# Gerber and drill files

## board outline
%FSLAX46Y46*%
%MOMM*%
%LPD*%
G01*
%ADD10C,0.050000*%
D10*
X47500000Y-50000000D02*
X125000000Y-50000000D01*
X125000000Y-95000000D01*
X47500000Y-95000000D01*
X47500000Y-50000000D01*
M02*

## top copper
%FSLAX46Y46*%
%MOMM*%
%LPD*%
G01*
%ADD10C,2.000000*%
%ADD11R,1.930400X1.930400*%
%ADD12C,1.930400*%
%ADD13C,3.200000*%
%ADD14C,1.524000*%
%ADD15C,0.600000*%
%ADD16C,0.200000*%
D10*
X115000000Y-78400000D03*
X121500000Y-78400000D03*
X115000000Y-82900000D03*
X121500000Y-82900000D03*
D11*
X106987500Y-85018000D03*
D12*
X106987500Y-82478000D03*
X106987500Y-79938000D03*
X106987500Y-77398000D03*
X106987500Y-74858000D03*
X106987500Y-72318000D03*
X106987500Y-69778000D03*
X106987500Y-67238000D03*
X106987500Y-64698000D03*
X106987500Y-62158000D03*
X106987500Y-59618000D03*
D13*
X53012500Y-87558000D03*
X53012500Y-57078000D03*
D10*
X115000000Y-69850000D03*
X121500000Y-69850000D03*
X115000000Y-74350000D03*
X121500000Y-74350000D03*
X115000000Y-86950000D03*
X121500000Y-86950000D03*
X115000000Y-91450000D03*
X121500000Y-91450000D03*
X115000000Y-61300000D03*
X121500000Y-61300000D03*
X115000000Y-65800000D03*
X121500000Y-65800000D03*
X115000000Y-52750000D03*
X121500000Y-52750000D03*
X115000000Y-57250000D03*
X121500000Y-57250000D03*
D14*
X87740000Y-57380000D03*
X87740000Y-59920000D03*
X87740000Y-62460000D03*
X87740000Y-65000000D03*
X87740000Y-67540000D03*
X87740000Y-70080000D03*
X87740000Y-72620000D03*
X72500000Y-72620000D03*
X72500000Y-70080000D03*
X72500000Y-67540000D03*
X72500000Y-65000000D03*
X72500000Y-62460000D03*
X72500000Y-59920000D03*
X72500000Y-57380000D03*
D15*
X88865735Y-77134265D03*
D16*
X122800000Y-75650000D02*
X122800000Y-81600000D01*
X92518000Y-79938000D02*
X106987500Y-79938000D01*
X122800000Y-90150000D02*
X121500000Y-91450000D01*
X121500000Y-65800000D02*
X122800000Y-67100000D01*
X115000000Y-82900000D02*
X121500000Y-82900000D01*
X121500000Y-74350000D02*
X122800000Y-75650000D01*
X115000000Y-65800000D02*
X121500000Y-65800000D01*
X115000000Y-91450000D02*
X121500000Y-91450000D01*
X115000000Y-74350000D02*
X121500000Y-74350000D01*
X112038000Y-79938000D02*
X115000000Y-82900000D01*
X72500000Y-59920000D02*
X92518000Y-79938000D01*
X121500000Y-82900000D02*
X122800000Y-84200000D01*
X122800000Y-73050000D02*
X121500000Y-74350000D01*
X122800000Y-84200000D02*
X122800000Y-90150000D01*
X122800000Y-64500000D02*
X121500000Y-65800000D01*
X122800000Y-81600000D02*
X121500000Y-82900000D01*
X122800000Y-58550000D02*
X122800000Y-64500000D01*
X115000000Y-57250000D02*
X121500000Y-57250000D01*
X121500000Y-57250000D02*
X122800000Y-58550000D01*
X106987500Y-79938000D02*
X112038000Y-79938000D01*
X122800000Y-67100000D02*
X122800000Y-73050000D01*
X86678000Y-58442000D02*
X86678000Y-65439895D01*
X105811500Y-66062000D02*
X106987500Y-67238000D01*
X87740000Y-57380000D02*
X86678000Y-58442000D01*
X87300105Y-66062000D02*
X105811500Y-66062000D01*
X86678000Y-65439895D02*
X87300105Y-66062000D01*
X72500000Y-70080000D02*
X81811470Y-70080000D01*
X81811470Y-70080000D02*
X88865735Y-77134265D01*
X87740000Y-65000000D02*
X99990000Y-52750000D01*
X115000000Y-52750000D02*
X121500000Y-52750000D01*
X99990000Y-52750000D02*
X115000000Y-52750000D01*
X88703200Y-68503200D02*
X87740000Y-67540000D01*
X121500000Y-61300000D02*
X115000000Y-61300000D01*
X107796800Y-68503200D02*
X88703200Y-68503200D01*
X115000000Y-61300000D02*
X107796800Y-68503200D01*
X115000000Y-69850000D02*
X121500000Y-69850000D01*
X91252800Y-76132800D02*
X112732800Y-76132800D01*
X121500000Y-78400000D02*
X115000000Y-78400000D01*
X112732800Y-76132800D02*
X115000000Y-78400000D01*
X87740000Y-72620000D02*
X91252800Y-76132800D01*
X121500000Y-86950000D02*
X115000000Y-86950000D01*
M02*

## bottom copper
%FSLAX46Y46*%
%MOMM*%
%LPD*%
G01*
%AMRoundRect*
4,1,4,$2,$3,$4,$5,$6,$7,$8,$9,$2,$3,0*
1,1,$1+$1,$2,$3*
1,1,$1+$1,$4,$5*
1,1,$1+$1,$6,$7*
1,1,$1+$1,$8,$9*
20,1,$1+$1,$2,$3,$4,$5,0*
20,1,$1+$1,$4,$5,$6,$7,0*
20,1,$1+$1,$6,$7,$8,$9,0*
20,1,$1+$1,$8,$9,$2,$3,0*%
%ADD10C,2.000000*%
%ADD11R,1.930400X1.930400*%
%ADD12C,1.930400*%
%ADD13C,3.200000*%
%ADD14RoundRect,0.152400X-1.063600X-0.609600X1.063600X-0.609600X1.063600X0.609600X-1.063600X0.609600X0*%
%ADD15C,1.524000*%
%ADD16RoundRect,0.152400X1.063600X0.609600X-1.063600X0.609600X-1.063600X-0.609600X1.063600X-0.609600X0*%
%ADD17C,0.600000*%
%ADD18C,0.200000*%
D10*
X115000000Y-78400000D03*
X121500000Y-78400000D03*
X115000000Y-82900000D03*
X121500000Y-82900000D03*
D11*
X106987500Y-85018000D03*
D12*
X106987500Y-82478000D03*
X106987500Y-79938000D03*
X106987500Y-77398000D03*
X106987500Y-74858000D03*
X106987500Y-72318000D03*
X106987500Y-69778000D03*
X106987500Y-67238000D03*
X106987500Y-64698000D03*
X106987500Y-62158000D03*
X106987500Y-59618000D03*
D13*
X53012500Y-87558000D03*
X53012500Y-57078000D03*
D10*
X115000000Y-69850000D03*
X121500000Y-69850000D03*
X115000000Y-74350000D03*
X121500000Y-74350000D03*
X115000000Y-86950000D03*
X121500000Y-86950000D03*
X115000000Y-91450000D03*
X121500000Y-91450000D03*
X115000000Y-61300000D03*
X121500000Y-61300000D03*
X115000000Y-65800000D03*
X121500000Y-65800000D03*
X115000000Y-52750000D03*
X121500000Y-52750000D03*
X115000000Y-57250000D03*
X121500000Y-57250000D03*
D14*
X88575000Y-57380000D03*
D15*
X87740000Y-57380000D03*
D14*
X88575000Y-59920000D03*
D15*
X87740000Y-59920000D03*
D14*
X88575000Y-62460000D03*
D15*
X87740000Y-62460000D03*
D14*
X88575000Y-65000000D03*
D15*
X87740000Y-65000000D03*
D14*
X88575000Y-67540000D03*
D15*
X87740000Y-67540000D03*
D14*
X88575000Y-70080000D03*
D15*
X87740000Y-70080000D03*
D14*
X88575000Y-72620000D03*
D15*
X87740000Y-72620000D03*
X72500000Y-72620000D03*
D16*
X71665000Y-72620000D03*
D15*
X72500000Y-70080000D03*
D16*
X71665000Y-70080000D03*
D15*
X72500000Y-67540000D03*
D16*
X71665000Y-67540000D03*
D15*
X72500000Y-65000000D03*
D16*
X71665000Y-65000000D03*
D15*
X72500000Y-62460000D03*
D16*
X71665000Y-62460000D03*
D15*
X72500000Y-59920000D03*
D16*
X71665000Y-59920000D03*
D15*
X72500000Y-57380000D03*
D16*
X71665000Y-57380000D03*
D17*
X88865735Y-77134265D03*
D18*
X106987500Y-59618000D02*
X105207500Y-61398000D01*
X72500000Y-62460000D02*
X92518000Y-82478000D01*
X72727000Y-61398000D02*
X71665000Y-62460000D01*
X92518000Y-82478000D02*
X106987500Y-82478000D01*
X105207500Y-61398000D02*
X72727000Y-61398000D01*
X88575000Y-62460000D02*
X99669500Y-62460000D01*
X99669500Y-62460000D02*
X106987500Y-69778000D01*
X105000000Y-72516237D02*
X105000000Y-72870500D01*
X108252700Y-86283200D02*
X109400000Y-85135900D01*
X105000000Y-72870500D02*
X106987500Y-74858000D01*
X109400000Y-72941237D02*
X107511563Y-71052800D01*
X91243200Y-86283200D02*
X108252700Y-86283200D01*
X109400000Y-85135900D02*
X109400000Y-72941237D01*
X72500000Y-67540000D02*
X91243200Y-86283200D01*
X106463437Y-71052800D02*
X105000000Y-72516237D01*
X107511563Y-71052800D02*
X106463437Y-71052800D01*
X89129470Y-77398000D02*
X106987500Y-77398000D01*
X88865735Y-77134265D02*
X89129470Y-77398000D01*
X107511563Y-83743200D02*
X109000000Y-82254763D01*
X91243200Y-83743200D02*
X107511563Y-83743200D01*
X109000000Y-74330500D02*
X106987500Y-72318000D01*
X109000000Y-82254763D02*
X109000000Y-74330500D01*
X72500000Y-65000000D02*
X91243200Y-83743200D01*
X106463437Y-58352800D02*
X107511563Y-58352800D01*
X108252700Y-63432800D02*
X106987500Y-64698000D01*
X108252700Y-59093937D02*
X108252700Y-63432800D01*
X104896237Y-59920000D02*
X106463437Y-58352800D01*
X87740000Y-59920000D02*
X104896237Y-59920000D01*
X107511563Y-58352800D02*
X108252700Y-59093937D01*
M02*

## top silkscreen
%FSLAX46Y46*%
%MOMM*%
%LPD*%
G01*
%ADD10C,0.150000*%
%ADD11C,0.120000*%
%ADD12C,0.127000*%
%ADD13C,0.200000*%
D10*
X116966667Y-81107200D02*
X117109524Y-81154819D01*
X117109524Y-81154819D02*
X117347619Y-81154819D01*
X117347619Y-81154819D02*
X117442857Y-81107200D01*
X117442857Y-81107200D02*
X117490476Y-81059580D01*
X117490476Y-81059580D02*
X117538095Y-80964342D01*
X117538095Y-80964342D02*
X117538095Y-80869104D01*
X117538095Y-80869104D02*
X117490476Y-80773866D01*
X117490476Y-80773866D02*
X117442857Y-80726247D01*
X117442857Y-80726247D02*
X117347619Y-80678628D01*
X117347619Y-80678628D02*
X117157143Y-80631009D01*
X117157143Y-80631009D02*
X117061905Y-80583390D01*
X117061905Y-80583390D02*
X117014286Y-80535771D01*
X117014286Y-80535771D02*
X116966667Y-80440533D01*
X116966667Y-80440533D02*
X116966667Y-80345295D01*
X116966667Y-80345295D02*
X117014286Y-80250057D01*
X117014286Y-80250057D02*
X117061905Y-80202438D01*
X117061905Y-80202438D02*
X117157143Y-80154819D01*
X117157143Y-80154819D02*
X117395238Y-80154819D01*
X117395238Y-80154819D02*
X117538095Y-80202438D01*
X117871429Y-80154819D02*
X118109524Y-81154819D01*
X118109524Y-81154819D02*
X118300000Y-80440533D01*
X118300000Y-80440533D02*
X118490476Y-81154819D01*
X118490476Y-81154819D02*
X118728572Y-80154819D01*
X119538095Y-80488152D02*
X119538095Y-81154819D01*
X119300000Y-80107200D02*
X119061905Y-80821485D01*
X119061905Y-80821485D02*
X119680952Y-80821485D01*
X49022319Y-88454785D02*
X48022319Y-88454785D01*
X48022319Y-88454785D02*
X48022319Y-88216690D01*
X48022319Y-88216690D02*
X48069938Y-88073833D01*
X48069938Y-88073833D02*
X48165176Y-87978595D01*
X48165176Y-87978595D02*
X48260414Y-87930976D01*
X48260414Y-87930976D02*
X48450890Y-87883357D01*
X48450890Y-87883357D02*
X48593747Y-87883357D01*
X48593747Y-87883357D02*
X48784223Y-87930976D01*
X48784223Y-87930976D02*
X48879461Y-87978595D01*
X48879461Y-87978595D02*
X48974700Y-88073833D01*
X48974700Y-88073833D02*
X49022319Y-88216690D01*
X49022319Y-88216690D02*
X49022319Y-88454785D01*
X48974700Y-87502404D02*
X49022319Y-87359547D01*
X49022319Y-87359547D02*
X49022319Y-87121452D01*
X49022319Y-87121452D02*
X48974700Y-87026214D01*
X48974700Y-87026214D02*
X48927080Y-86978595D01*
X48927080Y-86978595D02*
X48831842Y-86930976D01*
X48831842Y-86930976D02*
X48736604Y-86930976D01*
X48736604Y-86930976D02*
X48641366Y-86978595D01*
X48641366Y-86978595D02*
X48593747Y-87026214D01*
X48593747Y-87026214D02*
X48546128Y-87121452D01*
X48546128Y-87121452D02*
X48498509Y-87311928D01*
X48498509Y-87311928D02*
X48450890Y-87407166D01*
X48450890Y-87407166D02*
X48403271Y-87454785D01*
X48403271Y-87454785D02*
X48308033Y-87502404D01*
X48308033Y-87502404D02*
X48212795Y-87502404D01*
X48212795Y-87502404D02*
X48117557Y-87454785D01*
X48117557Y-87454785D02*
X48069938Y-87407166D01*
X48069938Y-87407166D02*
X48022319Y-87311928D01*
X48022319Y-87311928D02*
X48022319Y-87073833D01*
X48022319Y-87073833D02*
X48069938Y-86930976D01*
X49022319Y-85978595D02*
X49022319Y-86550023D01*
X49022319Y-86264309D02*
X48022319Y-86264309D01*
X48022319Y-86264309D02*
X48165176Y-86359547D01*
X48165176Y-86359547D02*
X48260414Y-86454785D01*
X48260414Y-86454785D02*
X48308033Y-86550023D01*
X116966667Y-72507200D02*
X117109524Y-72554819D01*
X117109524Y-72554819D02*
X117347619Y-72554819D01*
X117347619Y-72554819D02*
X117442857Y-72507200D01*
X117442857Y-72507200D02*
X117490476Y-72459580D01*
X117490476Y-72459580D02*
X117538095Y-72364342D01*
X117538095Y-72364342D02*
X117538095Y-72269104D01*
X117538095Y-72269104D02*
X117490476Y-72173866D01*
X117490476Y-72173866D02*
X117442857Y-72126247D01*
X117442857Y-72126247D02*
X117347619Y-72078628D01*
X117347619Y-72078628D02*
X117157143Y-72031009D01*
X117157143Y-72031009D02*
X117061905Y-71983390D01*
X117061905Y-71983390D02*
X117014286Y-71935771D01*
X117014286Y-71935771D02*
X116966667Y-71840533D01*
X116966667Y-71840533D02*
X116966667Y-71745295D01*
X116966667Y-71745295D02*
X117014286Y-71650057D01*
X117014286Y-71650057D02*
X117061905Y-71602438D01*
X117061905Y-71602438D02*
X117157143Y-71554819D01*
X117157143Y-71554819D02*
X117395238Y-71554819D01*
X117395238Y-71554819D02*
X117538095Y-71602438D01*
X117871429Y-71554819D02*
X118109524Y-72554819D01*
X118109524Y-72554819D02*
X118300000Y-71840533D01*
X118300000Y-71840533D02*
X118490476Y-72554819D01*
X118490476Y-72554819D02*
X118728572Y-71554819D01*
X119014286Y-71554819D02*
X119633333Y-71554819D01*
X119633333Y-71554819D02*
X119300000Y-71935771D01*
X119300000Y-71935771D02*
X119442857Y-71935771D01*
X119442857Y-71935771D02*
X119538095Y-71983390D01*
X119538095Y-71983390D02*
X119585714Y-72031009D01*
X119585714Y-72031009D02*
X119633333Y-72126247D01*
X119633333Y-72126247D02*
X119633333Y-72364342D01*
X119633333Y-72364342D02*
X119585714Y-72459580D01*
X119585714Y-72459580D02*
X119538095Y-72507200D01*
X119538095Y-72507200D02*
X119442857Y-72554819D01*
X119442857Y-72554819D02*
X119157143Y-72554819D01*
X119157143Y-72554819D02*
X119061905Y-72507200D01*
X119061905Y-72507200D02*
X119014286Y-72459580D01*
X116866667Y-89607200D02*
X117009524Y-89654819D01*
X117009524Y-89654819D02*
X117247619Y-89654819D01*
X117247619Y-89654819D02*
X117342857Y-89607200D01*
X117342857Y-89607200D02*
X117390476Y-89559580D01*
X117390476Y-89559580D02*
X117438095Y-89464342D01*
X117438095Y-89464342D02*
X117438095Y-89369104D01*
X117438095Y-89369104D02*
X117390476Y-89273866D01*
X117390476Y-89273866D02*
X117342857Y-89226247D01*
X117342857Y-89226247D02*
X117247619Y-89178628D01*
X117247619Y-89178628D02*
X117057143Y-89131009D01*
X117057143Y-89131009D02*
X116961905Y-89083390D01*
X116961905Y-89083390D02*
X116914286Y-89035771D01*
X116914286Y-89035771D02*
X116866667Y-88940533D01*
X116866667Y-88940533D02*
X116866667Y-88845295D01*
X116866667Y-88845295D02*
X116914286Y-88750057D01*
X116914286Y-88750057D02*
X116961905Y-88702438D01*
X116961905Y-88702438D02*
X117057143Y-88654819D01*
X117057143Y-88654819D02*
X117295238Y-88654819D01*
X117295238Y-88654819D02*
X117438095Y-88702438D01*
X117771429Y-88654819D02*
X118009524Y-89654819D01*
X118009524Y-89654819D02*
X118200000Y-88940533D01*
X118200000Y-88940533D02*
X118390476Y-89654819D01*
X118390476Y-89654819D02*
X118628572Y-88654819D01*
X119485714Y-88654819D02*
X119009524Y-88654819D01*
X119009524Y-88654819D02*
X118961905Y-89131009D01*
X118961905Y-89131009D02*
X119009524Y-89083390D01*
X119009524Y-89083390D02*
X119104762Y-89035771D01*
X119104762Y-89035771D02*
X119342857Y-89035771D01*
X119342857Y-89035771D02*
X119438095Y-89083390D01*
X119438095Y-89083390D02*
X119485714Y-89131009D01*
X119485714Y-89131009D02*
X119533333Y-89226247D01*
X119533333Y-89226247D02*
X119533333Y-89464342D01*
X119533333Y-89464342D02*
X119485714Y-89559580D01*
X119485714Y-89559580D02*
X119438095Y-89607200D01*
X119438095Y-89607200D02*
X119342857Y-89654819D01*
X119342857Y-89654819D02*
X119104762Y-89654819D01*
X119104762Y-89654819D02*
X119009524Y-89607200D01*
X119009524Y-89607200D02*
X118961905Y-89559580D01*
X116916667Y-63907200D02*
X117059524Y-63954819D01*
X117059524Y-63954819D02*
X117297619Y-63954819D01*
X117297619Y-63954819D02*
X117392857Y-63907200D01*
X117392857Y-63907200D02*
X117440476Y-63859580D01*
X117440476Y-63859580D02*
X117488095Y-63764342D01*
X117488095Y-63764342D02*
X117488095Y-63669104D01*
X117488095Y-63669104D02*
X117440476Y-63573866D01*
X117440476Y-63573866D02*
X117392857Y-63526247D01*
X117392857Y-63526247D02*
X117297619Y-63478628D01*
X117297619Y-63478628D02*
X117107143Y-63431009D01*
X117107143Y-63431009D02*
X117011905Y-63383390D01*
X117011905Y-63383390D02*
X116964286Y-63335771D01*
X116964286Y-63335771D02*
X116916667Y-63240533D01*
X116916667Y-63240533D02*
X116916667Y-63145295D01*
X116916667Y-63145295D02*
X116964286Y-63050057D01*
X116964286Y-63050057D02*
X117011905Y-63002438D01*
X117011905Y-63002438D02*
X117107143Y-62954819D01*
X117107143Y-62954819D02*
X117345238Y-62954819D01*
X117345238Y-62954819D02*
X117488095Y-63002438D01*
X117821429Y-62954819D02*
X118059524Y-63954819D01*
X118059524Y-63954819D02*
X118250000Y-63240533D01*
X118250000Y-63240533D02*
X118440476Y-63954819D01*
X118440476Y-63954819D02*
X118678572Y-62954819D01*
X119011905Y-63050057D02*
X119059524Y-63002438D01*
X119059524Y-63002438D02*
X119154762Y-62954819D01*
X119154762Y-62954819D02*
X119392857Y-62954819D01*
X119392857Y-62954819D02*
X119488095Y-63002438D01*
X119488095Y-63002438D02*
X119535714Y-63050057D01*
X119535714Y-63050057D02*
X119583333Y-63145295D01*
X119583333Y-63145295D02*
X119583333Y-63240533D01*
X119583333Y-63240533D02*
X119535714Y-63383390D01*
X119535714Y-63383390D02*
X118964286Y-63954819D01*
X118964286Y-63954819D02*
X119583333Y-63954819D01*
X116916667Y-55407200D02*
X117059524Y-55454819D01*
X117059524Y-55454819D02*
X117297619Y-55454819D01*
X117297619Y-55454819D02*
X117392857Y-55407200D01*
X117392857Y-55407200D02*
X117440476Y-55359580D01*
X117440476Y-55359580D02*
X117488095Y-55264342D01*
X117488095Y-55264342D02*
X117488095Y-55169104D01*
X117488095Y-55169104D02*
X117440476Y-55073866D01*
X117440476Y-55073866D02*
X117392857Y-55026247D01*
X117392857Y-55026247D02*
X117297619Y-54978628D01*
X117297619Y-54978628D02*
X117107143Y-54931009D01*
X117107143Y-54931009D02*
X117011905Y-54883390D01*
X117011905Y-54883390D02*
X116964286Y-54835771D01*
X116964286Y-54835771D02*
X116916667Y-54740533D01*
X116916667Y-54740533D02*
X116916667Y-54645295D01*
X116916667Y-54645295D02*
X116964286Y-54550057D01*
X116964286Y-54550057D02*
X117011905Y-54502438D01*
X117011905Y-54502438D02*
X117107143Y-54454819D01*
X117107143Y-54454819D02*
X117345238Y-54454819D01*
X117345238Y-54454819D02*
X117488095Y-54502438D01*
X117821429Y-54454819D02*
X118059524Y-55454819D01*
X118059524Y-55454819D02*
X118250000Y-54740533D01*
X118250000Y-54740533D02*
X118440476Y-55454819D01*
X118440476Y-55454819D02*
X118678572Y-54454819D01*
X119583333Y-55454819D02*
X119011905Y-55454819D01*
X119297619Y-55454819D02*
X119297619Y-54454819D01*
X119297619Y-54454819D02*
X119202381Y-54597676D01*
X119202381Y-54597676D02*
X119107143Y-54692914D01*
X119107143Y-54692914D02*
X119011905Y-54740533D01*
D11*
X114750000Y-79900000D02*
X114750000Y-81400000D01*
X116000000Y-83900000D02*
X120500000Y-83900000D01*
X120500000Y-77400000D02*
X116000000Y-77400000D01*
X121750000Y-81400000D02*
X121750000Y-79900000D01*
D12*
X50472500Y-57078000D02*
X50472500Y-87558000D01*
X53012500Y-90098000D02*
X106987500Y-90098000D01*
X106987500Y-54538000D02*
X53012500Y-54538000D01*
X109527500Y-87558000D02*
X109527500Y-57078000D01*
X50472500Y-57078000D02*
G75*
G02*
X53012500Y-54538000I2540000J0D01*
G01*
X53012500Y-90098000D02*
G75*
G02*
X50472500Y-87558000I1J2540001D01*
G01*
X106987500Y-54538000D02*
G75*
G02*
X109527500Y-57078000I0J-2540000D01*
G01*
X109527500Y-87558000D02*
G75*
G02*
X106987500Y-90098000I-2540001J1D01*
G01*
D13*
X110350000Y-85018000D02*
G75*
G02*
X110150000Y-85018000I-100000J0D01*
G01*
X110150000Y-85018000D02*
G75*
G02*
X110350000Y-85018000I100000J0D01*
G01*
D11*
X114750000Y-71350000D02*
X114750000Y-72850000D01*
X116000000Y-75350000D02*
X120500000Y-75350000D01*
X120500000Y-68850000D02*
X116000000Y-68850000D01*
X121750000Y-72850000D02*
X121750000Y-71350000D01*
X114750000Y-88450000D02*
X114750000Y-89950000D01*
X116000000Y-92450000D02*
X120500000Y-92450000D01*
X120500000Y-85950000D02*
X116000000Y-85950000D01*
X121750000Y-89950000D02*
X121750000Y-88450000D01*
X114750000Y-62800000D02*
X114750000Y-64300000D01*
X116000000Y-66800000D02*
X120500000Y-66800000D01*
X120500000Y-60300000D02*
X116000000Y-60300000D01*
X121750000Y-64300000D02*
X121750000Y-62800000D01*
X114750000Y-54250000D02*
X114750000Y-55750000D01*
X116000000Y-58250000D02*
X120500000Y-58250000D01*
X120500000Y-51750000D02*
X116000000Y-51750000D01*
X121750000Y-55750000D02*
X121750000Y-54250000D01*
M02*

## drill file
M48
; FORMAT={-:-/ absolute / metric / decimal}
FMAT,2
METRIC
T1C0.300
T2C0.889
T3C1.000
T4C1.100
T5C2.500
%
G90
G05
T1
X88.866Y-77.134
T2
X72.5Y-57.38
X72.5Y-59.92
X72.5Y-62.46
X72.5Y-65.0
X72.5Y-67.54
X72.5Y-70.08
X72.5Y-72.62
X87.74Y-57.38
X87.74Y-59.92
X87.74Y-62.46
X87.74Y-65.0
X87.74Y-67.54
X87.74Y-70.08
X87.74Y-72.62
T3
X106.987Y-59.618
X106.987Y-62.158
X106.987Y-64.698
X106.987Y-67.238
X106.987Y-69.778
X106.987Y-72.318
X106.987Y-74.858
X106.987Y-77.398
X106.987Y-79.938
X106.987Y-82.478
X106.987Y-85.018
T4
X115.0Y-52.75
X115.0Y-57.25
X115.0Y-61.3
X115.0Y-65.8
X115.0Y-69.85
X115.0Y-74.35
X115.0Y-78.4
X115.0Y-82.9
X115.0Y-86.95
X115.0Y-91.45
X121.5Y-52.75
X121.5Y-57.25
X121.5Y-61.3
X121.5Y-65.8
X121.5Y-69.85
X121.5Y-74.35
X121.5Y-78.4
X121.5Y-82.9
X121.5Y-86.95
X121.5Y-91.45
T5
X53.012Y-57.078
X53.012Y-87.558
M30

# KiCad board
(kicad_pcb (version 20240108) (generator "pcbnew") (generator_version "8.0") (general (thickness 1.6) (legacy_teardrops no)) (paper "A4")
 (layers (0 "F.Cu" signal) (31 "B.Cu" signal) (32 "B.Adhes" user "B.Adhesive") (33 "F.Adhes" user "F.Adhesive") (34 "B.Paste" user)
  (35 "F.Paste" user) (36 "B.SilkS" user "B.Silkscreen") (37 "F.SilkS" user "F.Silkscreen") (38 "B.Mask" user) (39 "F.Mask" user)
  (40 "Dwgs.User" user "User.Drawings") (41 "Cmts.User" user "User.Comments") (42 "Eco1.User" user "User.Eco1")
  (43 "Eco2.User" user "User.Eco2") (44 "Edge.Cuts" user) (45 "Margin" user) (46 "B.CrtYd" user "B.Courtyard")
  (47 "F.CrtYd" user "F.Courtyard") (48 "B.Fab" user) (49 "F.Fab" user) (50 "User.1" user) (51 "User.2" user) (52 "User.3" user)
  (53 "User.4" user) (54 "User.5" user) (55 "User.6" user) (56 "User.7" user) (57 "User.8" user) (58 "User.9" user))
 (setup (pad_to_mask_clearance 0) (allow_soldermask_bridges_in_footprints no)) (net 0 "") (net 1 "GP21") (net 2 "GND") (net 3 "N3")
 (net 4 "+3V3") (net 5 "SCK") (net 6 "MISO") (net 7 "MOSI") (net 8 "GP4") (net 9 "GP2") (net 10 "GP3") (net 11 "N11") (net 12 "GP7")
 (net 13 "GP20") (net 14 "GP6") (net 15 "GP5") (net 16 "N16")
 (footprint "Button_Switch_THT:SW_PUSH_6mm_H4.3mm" (layer "F.Cu") (at 115 78.4)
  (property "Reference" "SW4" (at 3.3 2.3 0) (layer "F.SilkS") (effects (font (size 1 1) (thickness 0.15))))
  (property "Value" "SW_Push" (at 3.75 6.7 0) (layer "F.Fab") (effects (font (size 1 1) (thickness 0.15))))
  (fp_line (start -0.25 1.5) (end -0.25 3) (stroke (width 0.12) (type solid)) (layer "F.SilkS"))
  (fp_line (start 1 5.5) (end 5.5 5.5) (stroke (width 0.12) (type solid)) (layer "F.SilkS"))
  (fp_line (start 5.5 -1) (end 1 -1) (stroke (width 0.12) (type solid)) (layer "F.SilkS"))
  (fp_line (start 6.75 3) (end 6.75 1.5) (stroke (width 0.12) (type solid)) (layer "F.SilkS"))
  (pad "1" thru_hole circle (at 0 0 90) (size 2 2) (drill 1.1) (layers "*.Cu" "*.Mask") (remove_unused_layers no) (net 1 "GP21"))
  (pad "1" thru_hole circle (at 6.5 0 90) (size 2 2) (drill 1.1) (layers "*.Cu" "*.Mask") (remove_unused_layers no) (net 1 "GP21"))
  (pad "2" thru_hole circle (at 0 4.5 90) (size 2 2) (drill 1.1) (layers "*.Cu" "*.Mask") (remove_unused_layers no) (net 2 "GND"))
  (pad "2" thru_hole circle (at 6.5 4.5 90) (size 2 2) (drill 1.1) (layers "*.Cu" "*.Mask") (remove_unused_layers no) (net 2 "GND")))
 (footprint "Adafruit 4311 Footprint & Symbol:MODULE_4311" (layer "F.Cu") (at 80 72.318 90)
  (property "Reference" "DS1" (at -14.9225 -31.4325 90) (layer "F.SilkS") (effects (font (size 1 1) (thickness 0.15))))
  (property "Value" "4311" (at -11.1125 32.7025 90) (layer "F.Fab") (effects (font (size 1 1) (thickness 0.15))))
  (fp_line (start 15.24 -29.5275) (end -15.24 -29.5275) (stroke (width 0.127) (type solid)) (layer "F.SilkS"))
  (fp_line (start -17.78 -26.9875) (end -17.78 26.9875) (stroke (width 0.127) (type solid)) (layer "F.SilkS"))
  (fp_line (start 17.78 26.9875) (end 17.78 -26.9875) (stroke (width 0.127) (type solid)) (layer "F.SilkS"))
  (fp_line (start -15.24 29.5275) (end 15.24 29.5275) (stroke (width 0.127) (type solid)) (layer "F.SilkS"))
  (fp_arc (start 15.24 -29.5275) (mid 17.036051 -28.783551) (end 17.78 -26.9875) (stroke (width 0.127) (type solid)) (layer "F.SilkS"))
  (fp_arc (start -17.78 -26.9875) (mid -17.036051 -28.783551) (end -15.24 -29.5275) (stroke (width 0.127) (type solid)) (layer "F.SilkS"))
  (fp_arc (start 17.78 26.9875) (mid 17.036051 28.783551) (end 15.24 29.5275) (stroke (width 0.127) (type solid)) (layer "F.SilkS"))
  (fp_arc (start -15.24 29.5275) (mid -17.036051 28.783551) (end -17.78 26.9875) (stroke (width 0.127) (type solid)) (layer "F.SilkS"))
  (fp_circle (center -12.7 30.25) (end -12.6 30.25) (stroke (width 0.2) (type solid)) (fill none) (layer "F.SilkS"))
  (pad "1" thru_hole rect (at -12.7 26.9875 90) (size 1.9304 1.9304) (drill 1) (layers "*.Cu" "*.Mask") (remove_unused_layers no)
   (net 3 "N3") (solder_mask_margin 0.102))
  (pad "2" thru_hole circle (at -10.16 26.9875 90) (size 1.9304 1.9304) (drill 1) (layers "*.Cu" "*.Mask") (remove_unused_layers no)
   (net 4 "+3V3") (solder_mask_margin 0.102))
  (pad "3" thru_hole circle (at -7.62 26.9875 90) (size 1.9304 1.9304) (drill 1) (layers "*.Cu" "*.Mask") (remove_unused_layers no)
   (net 2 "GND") (solder_mask_margin 0.102))
  (pad "4" thru_hole circle (at -5.08 26.9875 90) (size 1.9304 1.9304) (drill 1) (layers "*.Cu" "*.Mask") (remove_unused_layers no)
   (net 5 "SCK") (solder_mask_margin 0.102))
  (pad "5" thru_hole circle (at -2.54 26.9875 90) (size 1.9304 1.9304) (drill 1) (layers "*.Cu" "*.Mask") (remove_unused_layers no)
   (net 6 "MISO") (solder_mask_margin 0.102))
  (pad "6" thru_hole circle (at 0 26.9875 90) (size 1.9304 1.9304) (drill 1) (layers "*.Cu" "*.Mask") (remove_unused_layers no)
   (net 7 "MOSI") (solder_mask_margin 0.102))
  (pad "7" thru_hole circle (at 2.54 26.9875 90) (size 1.9304 1.9304) (drill 1) (layers "*.Cu" "*.Mask") (remove_unused_layers no)
   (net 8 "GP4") (solder_mask_margin 0.102))
  (pad "8" thru_hole circle (at 5.08 26.9875 90) (size 1.9304 1.9304) (drill 1) (layers "*.Cu" "*.Mask") (remove_unused_layers no)
   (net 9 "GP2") (solder_mask_margin 0.102))
  (pad "9" thru_hole circle (at 7.62 26.9875 90) (size 1.9304 1.9304) (drill 1) (layers "*.Cu" "*.Mask") (remove_unused_layers no)
   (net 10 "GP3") (solder_mask_margin 0.102))
  (pad "10" thru_hole circle (at 10.16 26.9875 90) (size 1.9304 1.9304) (drill 1) (layers "*.Cu" "*.Mask") (remove_unused_layers no)
   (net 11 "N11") (solder_mask_margin 0.102))
  (pad "11" thru_hole circle (at 12.7 26.9875 90) (size 1.9304 1.9304) (drill 1) (layers "*.Cu" "*.Mask") (remove_unused_layers no)
   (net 4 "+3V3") (solder_mask_margin 0.102))
  (pad "SH1" thru_hole circle (at -15.24 -26.9875 90) (size 3.2 3.2) (drill 2.5) (layers "*.Cu" "*.Mask") (remove_unused_layers no)
   (solder_mask_margin 0.102))
  (pad "SH2" thru_hole circle (at 15.24 -26.9875 90) (size 3.2 3.2) (drill 2.5) (layers "*.Cu" "*.Mask") (remove_unused_layers no)
   (solder_mask_margin 0.102))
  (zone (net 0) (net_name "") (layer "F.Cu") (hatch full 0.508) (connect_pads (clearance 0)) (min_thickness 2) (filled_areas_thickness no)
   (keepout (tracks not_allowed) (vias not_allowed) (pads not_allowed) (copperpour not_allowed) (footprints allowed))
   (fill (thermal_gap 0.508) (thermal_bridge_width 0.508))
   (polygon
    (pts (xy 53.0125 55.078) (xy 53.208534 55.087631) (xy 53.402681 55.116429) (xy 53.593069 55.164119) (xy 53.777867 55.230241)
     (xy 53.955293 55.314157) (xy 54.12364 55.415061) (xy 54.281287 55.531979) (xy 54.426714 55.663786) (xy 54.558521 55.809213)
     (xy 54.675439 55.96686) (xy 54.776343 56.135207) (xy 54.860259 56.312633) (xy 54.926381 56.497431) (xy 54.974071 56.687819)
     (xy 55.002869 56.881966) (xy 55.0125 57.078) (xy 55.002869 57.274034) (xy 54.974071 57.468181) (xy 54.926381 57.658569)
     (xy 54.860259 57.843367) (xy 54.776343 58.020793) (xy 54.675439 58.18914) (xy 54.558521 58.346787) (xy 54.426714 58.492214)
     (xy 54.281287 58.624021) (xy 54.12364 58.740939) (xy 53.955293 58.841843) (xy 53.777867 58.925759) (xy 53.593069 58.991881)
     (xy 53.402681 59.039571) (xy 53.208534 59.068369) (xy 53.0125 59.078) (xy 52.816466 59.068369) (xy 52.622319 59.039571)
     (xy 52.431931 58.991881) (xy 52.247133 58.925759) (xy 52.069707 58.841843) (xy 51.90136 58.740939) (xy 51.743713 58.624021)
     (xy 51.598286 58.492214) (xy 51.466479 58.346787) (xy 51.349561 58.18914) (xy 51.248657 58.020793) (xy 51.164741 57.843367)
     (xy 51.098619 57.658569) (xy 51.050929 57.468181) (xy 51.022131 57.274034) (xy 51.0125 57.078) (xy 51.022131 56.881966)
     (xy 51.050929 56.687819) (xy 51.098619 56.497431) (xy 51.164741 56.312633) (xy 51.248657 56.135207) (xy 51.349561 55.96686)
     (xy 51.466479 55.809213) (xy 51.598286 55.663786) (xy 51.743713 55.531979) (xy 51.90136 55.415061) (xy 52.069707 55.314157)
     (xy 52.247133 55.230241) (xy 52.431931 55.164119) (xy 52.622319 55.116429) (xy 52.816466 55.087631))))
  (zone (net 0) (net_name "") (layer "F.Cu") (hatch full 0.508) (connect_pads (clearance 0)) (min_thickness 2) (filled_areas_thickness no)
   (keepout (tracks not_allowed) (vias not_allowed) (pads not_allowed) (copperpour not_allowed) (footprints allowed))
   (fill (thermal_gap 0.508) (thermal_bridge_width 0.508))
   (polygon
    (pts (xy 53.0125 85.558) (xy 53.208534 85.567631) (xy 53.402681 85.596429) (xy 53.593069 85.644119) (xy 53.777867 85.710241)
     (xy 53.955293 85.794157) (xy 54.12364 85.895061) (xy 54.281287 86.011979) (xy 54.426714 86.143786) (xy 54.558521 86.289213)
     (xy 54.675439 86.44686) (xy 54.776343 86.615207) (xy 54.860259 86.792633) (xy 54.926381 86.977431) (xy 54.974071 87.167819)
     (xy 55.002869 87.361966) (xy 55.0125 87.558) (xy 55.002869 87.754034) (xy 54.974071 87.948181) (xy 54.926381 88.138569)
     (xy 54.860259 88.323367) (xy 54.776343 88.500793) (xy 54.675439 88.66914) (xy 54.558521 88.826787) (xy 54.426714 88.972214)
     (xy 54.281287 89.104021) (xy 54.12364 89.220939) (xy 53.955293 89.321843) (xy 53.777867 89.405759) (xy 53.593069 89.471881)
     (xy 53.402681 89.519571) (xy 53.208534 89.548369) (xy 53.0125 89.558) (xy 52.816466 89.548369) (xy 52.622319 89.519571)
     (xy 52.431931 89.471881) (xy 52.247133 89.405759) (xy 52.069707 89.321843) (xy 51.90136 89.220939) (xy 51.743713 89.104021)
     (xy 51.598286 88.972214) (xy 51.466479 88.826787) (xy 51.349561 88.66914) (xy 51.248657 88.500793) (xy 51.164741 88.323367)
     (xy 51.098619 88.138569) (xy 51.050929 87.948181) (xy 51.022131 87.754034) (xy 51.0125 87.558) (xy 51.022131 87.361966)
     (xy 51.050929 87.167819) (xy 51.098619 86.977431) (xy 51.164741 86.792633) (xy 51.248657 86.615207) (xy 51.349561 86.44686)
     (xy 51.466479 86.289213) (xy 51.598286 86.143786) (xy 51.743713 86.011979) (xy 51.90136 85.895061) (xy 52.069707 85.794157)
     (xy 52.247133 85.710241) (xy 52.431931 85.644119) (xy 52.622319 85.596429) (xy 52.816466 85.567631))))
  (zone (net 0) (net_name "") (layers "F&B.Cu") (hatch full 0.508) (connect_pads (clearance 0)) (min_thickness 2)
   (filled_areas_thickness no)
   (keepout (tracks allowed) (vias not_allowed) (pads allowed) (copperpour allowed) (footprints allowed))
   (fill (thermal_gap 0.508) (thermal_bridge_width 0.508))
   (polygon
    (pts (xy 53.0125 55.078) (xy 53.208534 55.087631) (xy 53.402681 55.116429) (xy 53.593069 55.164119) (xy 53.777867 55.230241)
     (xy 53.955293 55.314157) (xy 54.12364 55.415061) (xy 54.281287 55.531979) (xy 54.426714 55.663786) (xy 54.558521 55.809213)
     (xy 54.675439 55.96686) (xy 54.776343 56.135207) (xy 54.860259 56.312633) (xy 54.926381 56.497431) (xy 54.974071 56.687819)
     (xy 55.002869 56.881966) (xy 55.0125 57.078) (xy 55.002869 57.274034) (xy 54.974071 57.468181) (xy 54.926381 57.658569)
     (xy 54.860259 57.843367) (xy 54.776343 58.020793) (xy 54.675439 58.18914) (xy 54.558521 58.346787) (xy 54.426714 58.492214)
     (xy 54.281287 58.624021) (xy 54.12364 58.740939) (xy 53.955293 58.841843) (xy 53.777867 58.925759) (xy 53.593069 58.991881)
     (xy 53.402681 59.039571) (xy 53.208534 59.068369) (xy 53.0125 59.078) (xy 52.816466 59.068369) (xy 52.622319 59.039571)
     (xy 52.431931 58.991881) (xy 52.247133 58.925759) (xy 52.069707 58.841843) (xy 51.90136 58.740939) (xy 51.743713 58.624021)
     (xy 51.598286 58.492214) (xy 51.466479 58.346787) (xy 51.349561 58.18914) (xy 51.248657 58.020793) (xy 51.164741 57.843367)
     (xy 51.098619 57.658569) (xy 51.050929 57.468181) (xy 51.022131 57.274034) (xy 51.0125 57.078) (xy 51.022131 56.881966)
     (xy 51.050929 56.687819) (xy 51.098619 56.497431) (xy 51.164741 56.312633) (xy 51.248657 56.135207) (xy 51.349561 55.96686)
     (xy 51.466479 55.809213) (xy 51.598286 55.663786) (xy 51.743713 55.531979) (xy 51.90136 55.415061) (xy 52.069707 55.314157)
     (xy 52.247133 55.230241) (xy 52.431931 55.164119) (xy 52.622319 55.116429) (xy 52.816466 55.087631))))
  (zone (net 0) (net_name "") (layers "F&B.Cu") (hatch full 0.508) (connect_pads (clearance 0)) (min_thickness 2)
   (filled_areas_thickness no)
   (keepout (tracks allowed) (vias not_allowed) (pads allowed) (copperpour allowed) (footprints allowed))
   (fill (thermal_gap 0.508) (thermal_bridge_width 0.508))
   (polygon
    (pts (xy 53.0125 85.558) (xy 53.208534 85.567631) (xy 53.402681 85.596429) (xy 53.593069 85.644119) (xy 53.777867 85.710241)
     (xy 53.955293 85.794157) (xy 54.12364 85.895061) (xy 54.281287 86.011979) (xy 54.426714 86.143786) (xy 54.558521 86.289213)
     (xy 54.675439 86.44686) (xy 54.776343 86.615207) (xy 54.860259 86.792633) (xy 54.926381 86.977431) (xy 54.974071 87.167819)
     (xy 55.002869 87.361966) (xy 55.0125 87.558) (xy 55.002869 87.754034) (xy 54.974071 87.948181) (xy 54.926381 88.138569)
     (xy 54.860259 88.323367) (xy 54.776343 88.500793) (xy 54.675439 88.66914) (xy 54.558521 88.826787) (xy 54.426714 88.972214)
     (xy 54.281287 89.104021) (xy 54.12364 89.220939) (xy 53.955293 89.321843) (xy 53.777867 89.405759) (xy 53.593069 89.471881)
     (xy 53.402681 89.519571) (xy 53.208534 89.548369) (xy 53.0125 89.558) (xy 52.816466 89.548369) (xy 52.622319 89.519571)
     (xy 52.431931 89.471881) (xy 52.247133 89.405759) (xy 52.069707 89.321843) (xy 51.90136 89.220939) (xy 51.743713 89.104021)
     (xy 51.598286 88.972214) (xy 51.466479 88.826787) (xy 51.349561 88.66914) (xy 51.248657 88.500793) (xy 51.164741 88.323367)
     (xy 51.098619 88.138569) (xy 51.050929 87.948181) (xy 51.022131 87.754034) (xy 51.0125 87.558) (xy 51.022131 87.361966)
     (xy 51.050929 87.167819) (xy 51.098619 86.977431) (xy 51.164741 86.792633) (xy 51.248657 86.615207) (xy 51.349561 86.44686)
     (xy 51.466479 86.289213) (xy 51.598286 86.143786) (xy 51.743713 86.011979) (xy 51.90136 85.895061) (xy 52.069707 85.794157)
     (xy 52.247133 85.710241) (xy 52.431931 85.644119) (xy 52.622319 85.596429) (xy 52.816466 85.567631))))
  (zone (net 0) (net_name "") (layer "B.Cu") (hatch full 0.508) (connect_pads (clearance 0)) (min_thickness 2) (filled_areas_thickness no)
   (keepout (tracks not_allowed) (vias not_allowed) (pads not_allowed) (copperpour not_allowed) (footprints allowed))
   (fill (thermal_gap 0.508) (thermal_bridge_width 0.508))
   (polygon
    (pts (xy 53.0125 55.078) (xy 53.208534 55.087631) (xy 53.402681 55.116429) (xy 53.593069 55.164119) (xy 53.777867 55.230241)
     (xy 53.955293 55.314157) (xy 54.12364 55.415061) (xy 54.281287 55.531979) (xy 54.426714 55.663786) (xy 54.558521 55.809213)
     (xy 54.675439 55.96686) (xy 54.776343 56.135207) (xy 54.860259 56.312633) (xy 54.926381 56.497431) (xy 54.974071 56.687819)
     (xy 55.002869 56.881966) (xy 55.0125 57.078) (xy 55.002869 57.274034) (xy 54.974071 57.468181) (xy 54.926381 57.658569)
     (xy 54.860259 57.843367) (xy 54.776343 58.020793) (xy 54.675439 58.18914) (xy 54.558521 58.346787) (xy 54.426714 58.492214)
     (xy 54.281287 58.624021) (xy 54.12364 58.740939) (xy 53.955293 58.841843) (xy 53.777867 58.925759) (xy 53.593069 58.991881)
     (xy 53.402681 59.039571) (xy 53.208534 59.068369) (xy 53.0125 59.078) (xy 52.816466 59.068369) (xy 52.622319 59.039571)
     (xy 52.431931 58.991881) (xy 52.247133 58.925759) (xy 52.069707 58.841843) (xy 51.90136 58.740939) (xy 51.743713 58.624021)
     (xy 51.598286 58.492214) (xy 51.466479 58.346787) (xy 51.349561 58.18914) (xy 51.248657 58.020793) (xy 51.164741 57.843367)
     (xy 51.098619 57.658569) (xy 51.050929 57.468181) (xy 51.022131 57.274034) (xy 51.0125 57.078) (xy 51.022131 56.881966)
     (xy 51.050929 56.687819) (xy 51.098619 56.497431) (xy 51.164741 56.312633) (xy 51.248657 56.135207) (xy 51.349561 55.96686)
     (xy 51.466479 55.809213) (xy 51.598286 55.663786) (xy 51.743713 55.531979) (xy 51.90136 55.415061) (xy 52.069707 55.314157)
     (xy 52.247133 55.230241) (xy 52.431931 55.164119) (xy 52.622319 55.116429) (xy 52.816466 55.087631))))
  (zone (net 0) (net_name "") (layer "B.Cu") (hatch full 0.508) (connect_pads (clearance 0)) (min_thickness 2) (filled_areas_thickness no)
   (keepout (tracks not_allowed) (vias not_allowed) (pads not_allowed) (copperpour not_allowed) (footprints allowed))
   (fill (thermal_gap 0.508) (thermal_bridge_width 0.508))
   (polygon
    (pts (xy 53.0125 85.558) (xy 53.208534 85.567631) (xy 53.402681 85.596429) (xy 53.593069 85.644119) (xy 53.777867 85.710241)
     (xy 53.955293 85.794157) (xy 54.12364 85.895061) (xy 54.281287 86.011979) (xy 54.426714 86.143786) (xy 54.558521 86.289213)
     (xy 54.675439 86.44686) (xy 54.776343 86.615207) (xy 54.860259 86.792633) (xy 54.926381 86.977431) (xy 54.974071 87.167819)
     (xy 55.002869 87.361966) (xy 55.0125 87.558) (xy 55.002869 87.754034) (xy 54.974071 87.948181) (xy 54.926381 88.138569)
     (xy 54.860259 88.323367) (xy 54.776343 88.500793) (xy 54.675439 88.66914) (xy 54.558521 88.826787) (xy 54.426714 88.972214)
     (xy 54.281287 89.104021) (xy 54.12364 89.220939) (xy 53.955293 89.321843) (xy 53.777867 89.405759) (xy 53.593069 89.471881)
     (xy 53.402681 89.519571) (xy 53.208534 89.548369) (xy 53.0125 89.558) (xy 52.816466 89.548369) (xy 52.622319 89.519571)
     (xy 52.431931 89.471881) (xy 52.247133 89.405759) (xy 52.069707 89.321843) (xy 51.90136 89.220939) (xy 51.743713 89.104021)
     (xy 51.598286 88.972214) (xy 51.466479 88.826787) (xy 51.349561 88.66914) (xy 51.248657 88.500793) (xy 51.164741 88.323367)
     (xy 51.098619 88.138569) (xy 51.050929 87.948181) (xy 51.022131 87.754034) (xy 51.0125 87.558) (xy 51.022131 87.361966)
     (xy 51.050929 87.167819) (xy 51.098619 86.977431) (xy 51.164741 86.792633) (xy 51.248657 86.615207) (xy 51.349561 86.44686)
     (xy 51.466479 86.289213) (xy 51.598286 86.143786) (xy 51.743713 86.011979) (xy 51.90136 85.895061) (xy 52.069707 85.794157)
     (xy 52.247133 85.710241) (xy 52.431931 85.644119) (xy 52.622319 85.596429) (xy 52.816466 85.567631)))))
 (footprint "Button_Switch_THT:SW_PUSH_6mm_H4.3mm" (layer "F.Cu") (at 115 69.85)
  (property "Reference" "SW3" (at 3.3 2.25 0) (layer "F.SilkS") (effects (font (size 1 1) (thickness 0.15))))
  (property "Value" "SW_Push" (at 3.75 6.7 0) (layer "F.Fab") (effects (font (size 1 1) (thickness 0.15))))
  (fp_line (start -0.25 1.5) (end -0.25 3) (stroke (width 0.12) (type solid)) (layer "F.SilkS"))
  (fp_line (start 1 5.5) (end 5.5 5.5) (stroke (width 0.12) (type solid)) (layer "F.SilkS"))
  (fp_line (start 5.5 -1) (end 1 -1) (stroke (width 0.12) (type solid)) (layer "F.SilkS"))
  (fp_line (start 6.75 3) (end 6.75 1.5) (stroke (width 0.12) (type solid)) (layer "F.SilkS"))
  (pad "1" thru_hole circle (at 0 0 90) (size 2 2) (drill 1.1) (layers "*.Cu" "*.Mask") (remove_unused_layers no) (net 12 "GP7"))
  (pad "1" thru_hole circle (at 6.5 0 90) (size 2 2) (drill 1.1) (layers "*.Cu" "*.Mask") (remove_unused_layers no) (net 12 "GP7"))
  (pad "2" thru_hole circle (at 0 4.5 90) (size 2 2) (drill 1.1) (layers "*.Cu" "*.Mask") (remove_unused_layers no) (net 2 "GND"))
  (pad "2" thru_hole circle (at 6.5 4.5 90) (size 2 2) (drill 1.1) (layers "*.Cu" "*.Mask") (remove_unused_layers no) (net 2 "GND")))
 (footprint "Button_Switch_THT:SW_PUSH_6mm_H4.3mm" (layer "F.Cu") (at 115 86.95)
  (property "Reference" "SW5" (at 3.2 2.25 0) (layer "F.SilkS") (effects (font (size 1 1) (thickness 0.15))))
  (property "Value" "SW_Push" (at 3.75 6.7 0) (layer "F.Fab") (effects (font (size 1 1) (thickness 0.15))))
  (fp_line (start -0.25 1.5) (end -0.25 3) (stroke (width 0.12) (type solid)) (layer "F.SilkS"))
  (fp_line (start 1 5.5) (end 5.5 5.5) (stroke (width 0.12) (type solid)) (layer "F.SilkS"))
  (fp_line (start 5.5 -1) (end 1 -1) (stroke (width 0.12) (type solid)) (layer "F.SilkS"))
  (fp_line (start 6.75 3) (end 6.75 1.5) (stroke (width 0.12) (type solid)) (layer "F.SilkS"))
  (pad "1" thru_hole circle (at 0 0 90) (size 2 2) (drill 1.1) (layers "*.Cu" "*.Mask") (remove_unused_layers no) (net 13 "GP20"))
  (pad "1" thru_hole circle (at 6.5 0 90) (size 2 2) (drill 1.1) (layers "*.Cu" "*.Mask") (remove_unused_layers no) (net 13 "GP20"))
  (pad "2" thru_hole circle (at 0 4.5 90) (size 2 2) (drill 1.1) (layers "*.Cu" "*.Mask") (remove_unused_layers no) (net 2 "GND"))
  (pad "2" thru_hole circle (at 6.5 4.5 90) (size 2 2) (drill 1.1) (layers "*.Cu" "*.Mask") (remove_unused_layers no) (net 2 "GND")))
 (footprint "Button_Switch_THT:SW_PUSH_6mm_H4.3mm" (layer "F.Cu") (at 115 61.3)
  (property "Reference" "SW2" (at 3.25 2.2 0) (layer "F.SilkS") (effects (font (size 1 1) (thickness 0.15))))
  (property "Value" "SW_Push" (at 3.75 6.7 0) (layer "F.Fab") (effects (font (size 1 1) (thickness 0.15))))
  (fp_line (start -0.25 1.5) (end -0.25 3) (stroke (width 0.12) (type solid)) (layer "F.SilkS"))
  (fp_line (start 1 5.5) (end 5.5 5.5) (stroke (width 0.12) (type solid)) (layer "F.SilkS"))
  (fp_line (start 5.5 -1) (end 1 -1) (stroke (width 0.12) (type solid)) (layer "F.SilkS"))
  (fp_line (start 6.75 3) (end 6.75 1.5) (stroke (width 0.12) (type solid)) (layer "F.SilkS"))
  (pad "1" thru_hole circle (at 0 0 90) (size 2 2) (drill 1.1) (layers "*.Cu" "*.Mask") (remove_unused_layers no) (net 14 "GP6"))
  (pad "1" thru_hole circle (at 6.5 0 90) (size 2 2) (drill 1.1) (layers "*.Cu" "*.Mask") (remove_unused_layers no) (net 14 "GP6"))
  (pad "2" thru_hole circle (at 0 4.5 90) (size 2 2) (drill 1.1) (layers "*.Cu" "*.Mask") (remove_unused_layers no) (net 2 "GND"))
  (pad "2" thru_hole circle (at 6.5 4.5 90) (size 2 2) (drill 1.1) (layers "*.Cu" "*.Mask") (remove_unused_layers no) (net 2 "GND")))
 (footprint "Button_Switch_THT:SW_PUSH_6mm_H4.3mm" (layer "F.Cu") (at 115 52.75)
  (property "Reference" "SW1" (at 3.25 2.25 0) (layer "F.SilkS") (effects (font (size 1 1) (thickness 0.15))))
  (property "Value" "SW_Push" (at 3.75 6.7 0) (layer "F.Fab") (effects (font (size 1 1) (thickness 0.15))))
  (fp_line (start -0.25 1.5) (end -0.25 3) (stroke (width 0.12) (type solid)) (layer "F.SilkS"))
  (fp_line (start 1 5.5) (end 5.5 5.5) (stroke (width 0.12) (type solid)) (layer "F.SilkS"))
  (fp_line (start 5.5 -1) (end 1 -1) (stroke (width 0.12) (type solid)) (layer "F.SilkS"))
  (fp_line (start 6.75 3) (end 6.75 1.5) (stroke (width 0.12) (type solid)) (layer "F.SilkS"))
  (pad "1" thru_hole circle (at 0 0 90) (size 2 2) (drill 1.1) (layers "*.Cu" "*.Mask") (remove_unused_layers no) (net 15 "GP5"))
  (pad "1" thru_hole circle (at 6.5 0 90) (size 2 2) (drill 1.1) (layers "*.Cu" "*.Mask") (remove_unused_layers no) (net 15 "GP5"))
  (pad "2" thru_hole circle (at 0 4.5 90) (size 2 2) (drill 1.1) (layers "*.Cu" "*.Mask") (remove_unused_layers no) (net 2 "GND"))
  (pad "2" thru_hole circle (at 6.5 4.5 90) (size 2 2) (drill 1.1) (layers "*.Cu" "*.Mask") (remove_unused_layers no) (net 2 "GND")))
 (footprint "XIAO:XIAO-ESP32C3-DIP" (layer "B.Cu") (at 80 65 180)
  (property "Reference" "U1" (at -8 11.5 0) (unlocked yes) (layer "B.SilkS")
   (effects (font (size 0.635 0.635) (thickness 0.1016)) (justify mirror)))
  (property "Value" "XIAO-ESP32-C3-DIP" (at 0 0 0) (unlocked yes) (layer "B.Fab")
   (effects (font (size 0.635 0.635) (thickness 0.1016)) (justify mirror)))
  (pad "1" smd roundrect (at -8.575 7.62) (size 2.432 1.524) (layers "B.Cu" "B.Mask") (roundrect_rratio 0.1) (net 9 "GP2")
   (thermal_bridge_angle 45))
  (pad "1" thru_hole circle (at -7.74 7.62) (size 1.524 1.524) (drill 0.889) (layers "*.Cu" "*.Mask") (remove_unused_layers no)
   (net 9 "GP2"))
  (pad "2" smd roundrect (at -8.575 5.08) (size 2.432 1.524) (layers "B.Cu" "B.Mask") (roundrect_rratio 0.1) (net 10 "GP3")
   (thermal_bridge_angle 45))
  (pad "2" thru_hole circle (at -7.74 5.08) (size 1.524 1.524) (drill 0.889) (layers "*.Cu" "*.Mask") (remove_unused_layers no)
   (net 10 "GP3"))
  (pad "3" smd roundrect (at -8.575 2.54) (size 2.432 1.524) (layers "B.Cu" "B.Mask") (roundrect_rratio 0.1) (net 8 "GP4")
   (thermal_bridge_angle 45))
  (pad "3" thru_hole circle (at -7.74 2.54) (size 1.524 1.524) (drill 0.889) (layers "*.Cu" "*.Mask") (remove_unused_layers no)
   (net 8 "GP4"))
  (pad "4" smd roundrect (at -8.575 0) (size 2.432 1.524) (layers "B.Cu" "B.Mask") (roundrect_rratio 0.1) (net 15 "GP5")
   (thermal_bridge_angle 45))
  (pad "4" thru_hole circle (at -7.74 0) (size 1.524 1.524) (drill 0.889) (layers "*.Cu" "*.Mask") (remove_unused_layers no) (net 15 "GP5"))
  (pad "5" smd roundrect (at -8.575 -2.54) (size 2.432 1.524) (layers "B.Cu" "B.Mask") (roundrect_rratio 0.1) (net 14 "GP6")
   (thermal_bridge_angle 45))
  (pad "5" thru_hole circle (at -7.74 -2.54) (size 1.524 1.524) (drill 0.889) (layers "*.Cu" "*.Mask") (remove_unused_layers no)
   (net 14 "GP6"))
  (pad "6" smd roundrect (at -8.575 -5.08) (size 2.432 1.524) (layers "B.Cu" "B.Mask") (roundrect_rratio 0.1) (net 12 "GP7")
   (thermal_bridge_angle 45))
  (pad "6" thru_hole circle (at -7.74 -5.08) (size 1.524 1.524) (drill 0.889) (layers "*.Cu" "*.Mask") (remove_unused_layers no)
   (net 12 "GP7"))
  (pad "7" smd roundrect (at -8.575 -7.62) (size 2.432 1.524) (layers "B.Cu" "B.Mask") (roundrect_rratio 0.1) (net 1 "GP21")
   (thermal_bridge_angle 45))
  (pad "7" thru_hole circle (at -7.74 -7.62) (size 1.524 1.524) (drill 0.889) (layers "*.Cu" "*.Mask") (remove_unused_layers no)
   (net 1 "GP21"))
  (pad "8" thru_hole circle (at 7.5 -7.62 180) (size 1.524 1.524) (drill 0.889) (layers "*.Cu" "*.Mask") (remove_unused_layers no)
   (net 13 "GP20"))
  (pad "8" smd roundrect (at 8.335 -7.62 180) (size 2.432 1.524) (layers "B.Cu" "B.Mask") (roundrect_rratio 0.1) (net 13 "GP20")
   (thermal_bridge_angle 45))
  (pad "9" thru_hole circle (at 7.5 -5.08 180) (size 1.524 1.524) (drill 0.889) (layers "*.Cu" "*.Mask") (remove_unused_layers no)
   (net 5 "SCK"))
  (pad "9" smd roundrect (at 8.335 -5.08 180) (size 2.432 1.524) (layers "B.Cu" "B.Mask") (roundrect_rratio 0.1) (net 5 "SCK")
   (thermal_bridge_angle 45))
  (pad "10" thru_hole circle (at 7.5 -2.54 180) (size 1.524 1.524) (drill 0.889) (layers "*.Cu" "*.Mask") (remove_unused_layers no)
   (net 6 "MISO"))
  (pad "10" smd roundrect (at 8.335 -2.54 180) (size 2.432 1.524) (layers "B.Cu" "B.Mask") (roundrect_rratio 0.1) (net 6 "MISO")
   (thermal_bridge_angle 45))
  (pad "11" thru_hole circle (at 7.5 0 180) (size 1.524 1.524) (drill 0.889) (layers "*.Cu" "*.Mask") (remove_unused_layers no)
   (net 7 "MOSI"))
  (pad "11" smd roundrect (at 8.335 0 180) (size 2.432 1.524) (layers "B.Cu" "B.Mask") (roundrect_rratio 0.1) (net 7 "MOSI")
   (thermal_bridge_angle 45))
  (pad "12" thru_hole circle (at 7.5 2.54 180) (size 1.524 1.524) (drill 0.889) (layers "*.Cu" "*.Mask") (remove_unused_layers no)
   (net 4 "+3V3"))
  (pad "12" smd roundrect (at 8.335 2.54 180) (size 2.432 1.524) (layers "B.Cu" "B.Mask") (roundrect_rratio 0.1) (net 4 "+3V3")
   (thermal_bridge_angle 45))
  (pad "13" thru_hole circle (at 7.5 5.08 180) (size 1.524 1.524) (drill 0.889) (layers "*.Cu" "*.Mask") (remove_unused_layers no)
   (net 2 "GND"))
  (pad "13" smd roundrect (at 8.335 5.08 180) (size 2.432 1.524) (layers "B.Cu" "B.Mask") (roundrect_rratio 0.1) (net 2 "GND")
   (thermal_bridge_angle 45))
  (pad "14" thru_hole circle (at 7.5 7.62 180) (size 1.524 1.524) (drill 0.889) (layers "*.Cu" "*.Mask") (remove_unused_layers no)
   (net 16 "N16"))
  (pad "14" smd roundrect (at 8.335 7.62 180) (size 2.432 1.524) (layers "B.Cu" "B.Mask") (roundrect_rratio 0.1) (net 16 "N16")
   (thermal_bridge_angle 45)))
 (gr_rect (start 47.5 50) (end 125 95) (stroke (width 0.05) (type default)) (fill none) (layer "Edge.Cuts"))
 (segment (start 122.8 75.65) (end 122.8 81.6) (width 0.2) (layer "F.Cu") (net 2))
 (segment (start 92.518 79.938) (end 106.9875 79.938) (width 0.2) (layer "F.Cu") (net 2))
 (segment (start 122.8 90.15) (end 121.5 91.45) (width 0.2) (layer "F.Cu") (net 2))
 (segment (start 121.5 65.8) (end 122.8 67.1) (width 0.2) (layer "F.Cu") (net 2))
 (segment (start 115 82.9) (end 121.5 82.9) (width 0.2) (layer "F.Cu") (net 2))
 (segment (start 121.5 74.35) (end 122.8 75.65) (width 0.2) (layer "F.Cu") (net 2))
 (segment (start 115 65.8) (end 121.5 65.8) (width 0.2) (layer "F.Cu") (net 2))
 (segment (start 115 91.45) (end 121.5 91.45) (width 0.2) (layer "F.Cu") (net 2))
 (segment (start 115 74.35) (end 121.5 74.35) (width 0.2) (layer "F.Cu") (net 2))
 (segment (start 112.038 79.938) (end 115 82.9) (width 0.2) (layer "F.Cu") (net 2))
 (segment (start 72.5 59.92) (end 92.518 79.938) (width 0.2) (layer "F.Cu") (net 2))
 (segment (start 121.5 82.9) (end 122.8 84.2) (width 0.2) (layer "F.Cu") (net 2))
 (segment (start 122.8 73.05) (end 121.5 74.35) (width 0.2) (layer "F.Cu") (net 2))
 (segment (start 122.8 84.2) (end 122.8 90.15) (width 0.2) (layer "F.Cu") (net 2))
 (segment (start 122.8 64.5) (end 121.5 65.8) (width 0.2) (layer "F.Cu") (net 2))
 (segment (start 122.8 81.6) (end 121.5 82.9) (width 0.2) (layer "F.Cu") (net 2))
 (segment (start 122.8 58.55) (end 122.8 64.5) (width 0.2) (layer "F.Cu") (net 2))
 (segment (start 115 57.25) (end 121.5 57.25) (width 0.2) (layer "F.Cu") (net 2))
 (segment (start 121.5 57.25) (end 122.8 58.55) (width 0.2) (layer "F.Cu") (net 2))
 (segment (start 106.9875 79.938) (end 112.038 79.938) (width 0.2) (layer "F.Cu") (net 2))
 (segment (start 122.8 67.1) (end 122.8 73.05) (width 0.2) (layer "F.Cu") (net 2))
 (segment (start 106.9875 59.618) (end 105.2075 61.398) (width 0.2) (layer "B.Cu") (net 4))
 (segment (start 72.5 62.46) (end 92.518 82.478) (width 0.2) (layer "B.Cu") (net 4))
 (segment (start 72.727 61.398) (end 71.665 62.46) (width 0.2) (layer "B.Cu") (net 4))
 (segment (start 92.518 82.478) (end 106.9875 82.478) (width 0.2) (layer "B.Cu") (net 4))
 (segment (start 105.2075 61.398) (end 72.727 61.398) (width 0.2) (layer "B.Cu") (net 4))
 (segment (start 88.575 62.46) (end 99.6695 62.46) (width 0.2) (layer "B.Cu") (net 8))
 (segment (start 99.6695 62.46) (end 106.9875 69.778) (width 0.2) (layer "B.Cu") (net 8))
 (segment (start 105 72.516237) (end 105 72.8705) (width 0.2) (layer "B.Cu") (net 6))
 (segment (start 108.2527 86.2832) (end 109.4 85.1359) (width 0.2) (layer "B.Cu") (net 6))
 (segment (start 105 72.8705) (end 106.9875 74.858) (width 0.2) (layer "B.Cu") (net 6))
 (segment (start 109.4 72.941237) (end 107.511563 71.0528) (width 0.2) (layer "B.Cu") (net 6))
 (segment (start 91.2432 86.2832) (end 108.2527 86.2832) (width 0.2) (layer "B.Cu") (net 6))
 (segment (start 109.4 85.1359) (end 109.4 72.941237) (width 0.2) (layer "B.Cu") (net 6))
 (segment (start 72.5 67.54) (end 91.2432 86.2832) (width 0.2) (layer "B.Cu") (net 6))
 (segment (start 106.463437 71.0528) (end 105 72.516237) (width 0.2) (layer "B.Cu") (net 6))
 (segment (start 107.511563 71.0528) (end 106.463437 71.0528) (width 0.2) (layer "B.Cu") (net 6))
 (segment (start 86.678 58.442) (end 86.678 65.439895) (width 0.2) (layer "F.Cu") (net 9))
 (segment (start 105.8115 66.062) (end 106.9875 67.238) (width 0.2) (layer "F.Cu") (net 9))
 (segment (start 87.74 57.38) (end 86.678 58.442) (width 0.2) (layer "F.Cu") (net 9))
 (segment (start 87.300105 66.062) (end 105.8115 66.062) (width 0.2) (layer "F.Cu") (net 9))
 (segment (start 86.678 65.439895) (end 87.300105 66.062) (width 0.2) (layer "F.Cu") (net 9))
 (segment (start 72.5 70.08) (end 81.81147 70.08) (width 0.2) (layer "F.Cu") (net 5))
 (segment (start 81.81147 70.08) (end 88.865735 77.134265) (width 0.2) (layer "F.Cu") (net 5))
 (via (at 88.865735 77.134265) (size 0.6) (drill 0.3) (layers "F.Cu" "B.Cu") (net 5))
 (segment (start 89.12947 77.398) (end 106.9875 77.398) (width 0.2) (layer "B.Cu") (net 5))
 (segment (start 88.865735 77.134265) (end 89.12947 77.398) (width 0.2) (layer "B.Cu") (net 5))
 (segment (start 107.511563 83.7432) (end 109 82.254763) (width 0.2) (layer "B.Cu") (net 7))
 (segment (start 91.2432 83.7432) (end 107.511563 83.7432) (width 0.2) (layer "B.Cu") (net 7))
 (segment (start 109 74.3305) (end 106.9875 72.318) (width 0.2) (layer "B.Cu") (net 7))
 (segment (start 109 82.254763) (end 109 74.3305) (width 0.2) (layer "B.Cu") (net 7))
 (segment (start 72.5 65) (end 91.2432 83.7432) (width 0.2) (layer "B.Cu") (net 7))
 (segment (start 106.463437 58.3528) (end 107.511563 58.3528) (width 0.2) (layer "B.Cu") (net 10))
 (segment (start 108.2527 63.4328) (end 106.9875 64.698) (width 0.2) (layer "B.Cu") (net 10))
 (segment (start 108.2527 59.093937) (end 108.2527 63.4328) (width 0.2) (layer "B.Cu") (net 10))
 (segment (start 104.896237 59.92) (end 106.463437 58.3528) (width 0.2) (layer "B.Cu") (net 10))
 (segment (start 87.74 59.92) (end 104.896237 59.92) (width 0.2) (layer "B.Cu") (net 10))
 (segment (start 107.511563 58.3528) (end 108.2527 59.093937) (width 0.2) (layer "B.Cu") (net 10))
 (segment (start 87.74 65) (end 99.99 52.75) (width 0.2) (layer "F.Cu") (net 15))
 (segment (start 115 52.75) (end 121.5 52.75) (width 0.2) (layer "F.Cu") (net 15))
 (segment (start 99.99 52.75) (end 115 52.75) (width 0.2) (layer "F.Cu") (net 15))
 (segment (start 88.7032 68.5032) (end 87.74 67.54) (width 0.2) (layer "F.Cu") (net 14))
 (segment (start 121.5 61.3) (end 115 61.3) (width 0.2) (layer "F.Cu") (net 14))
 (segment (start 107.7968 68.5032) (end 88.7032 68.5032) (width 0.2) (layer "F.Cu") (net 14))
 (segment (start 115 61.3) (end 107.7968 68.5032) (width 0.2) (layer "F.Cu") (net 14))
 (segment (start 115 69.85) (end 121.5 69.85) (width 0.2) (layer "F.Cu") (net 12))
 (segment (start 91.2528 76.1328) (end 112.7328 76.1328) (width 0.2) (layer "F.Cu") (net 1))
 (segment (start 121.5 78.4) (end 115 78.4) (width 0.2) (layer "F.Cu") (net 1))
 (segment (start 112.7328 76.1328) (end 115 78.4) (width 0.2) (layer "F.Cu") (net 1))
 (segment (start 87.74 72.62) (end 91.2528 76.1328) (width 0.2) (layer "F.Cu") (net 1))
 (segment (start 121.5 86.95) (end 115 86.95) (width 0.2) (layer "F.Cu") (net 13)))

